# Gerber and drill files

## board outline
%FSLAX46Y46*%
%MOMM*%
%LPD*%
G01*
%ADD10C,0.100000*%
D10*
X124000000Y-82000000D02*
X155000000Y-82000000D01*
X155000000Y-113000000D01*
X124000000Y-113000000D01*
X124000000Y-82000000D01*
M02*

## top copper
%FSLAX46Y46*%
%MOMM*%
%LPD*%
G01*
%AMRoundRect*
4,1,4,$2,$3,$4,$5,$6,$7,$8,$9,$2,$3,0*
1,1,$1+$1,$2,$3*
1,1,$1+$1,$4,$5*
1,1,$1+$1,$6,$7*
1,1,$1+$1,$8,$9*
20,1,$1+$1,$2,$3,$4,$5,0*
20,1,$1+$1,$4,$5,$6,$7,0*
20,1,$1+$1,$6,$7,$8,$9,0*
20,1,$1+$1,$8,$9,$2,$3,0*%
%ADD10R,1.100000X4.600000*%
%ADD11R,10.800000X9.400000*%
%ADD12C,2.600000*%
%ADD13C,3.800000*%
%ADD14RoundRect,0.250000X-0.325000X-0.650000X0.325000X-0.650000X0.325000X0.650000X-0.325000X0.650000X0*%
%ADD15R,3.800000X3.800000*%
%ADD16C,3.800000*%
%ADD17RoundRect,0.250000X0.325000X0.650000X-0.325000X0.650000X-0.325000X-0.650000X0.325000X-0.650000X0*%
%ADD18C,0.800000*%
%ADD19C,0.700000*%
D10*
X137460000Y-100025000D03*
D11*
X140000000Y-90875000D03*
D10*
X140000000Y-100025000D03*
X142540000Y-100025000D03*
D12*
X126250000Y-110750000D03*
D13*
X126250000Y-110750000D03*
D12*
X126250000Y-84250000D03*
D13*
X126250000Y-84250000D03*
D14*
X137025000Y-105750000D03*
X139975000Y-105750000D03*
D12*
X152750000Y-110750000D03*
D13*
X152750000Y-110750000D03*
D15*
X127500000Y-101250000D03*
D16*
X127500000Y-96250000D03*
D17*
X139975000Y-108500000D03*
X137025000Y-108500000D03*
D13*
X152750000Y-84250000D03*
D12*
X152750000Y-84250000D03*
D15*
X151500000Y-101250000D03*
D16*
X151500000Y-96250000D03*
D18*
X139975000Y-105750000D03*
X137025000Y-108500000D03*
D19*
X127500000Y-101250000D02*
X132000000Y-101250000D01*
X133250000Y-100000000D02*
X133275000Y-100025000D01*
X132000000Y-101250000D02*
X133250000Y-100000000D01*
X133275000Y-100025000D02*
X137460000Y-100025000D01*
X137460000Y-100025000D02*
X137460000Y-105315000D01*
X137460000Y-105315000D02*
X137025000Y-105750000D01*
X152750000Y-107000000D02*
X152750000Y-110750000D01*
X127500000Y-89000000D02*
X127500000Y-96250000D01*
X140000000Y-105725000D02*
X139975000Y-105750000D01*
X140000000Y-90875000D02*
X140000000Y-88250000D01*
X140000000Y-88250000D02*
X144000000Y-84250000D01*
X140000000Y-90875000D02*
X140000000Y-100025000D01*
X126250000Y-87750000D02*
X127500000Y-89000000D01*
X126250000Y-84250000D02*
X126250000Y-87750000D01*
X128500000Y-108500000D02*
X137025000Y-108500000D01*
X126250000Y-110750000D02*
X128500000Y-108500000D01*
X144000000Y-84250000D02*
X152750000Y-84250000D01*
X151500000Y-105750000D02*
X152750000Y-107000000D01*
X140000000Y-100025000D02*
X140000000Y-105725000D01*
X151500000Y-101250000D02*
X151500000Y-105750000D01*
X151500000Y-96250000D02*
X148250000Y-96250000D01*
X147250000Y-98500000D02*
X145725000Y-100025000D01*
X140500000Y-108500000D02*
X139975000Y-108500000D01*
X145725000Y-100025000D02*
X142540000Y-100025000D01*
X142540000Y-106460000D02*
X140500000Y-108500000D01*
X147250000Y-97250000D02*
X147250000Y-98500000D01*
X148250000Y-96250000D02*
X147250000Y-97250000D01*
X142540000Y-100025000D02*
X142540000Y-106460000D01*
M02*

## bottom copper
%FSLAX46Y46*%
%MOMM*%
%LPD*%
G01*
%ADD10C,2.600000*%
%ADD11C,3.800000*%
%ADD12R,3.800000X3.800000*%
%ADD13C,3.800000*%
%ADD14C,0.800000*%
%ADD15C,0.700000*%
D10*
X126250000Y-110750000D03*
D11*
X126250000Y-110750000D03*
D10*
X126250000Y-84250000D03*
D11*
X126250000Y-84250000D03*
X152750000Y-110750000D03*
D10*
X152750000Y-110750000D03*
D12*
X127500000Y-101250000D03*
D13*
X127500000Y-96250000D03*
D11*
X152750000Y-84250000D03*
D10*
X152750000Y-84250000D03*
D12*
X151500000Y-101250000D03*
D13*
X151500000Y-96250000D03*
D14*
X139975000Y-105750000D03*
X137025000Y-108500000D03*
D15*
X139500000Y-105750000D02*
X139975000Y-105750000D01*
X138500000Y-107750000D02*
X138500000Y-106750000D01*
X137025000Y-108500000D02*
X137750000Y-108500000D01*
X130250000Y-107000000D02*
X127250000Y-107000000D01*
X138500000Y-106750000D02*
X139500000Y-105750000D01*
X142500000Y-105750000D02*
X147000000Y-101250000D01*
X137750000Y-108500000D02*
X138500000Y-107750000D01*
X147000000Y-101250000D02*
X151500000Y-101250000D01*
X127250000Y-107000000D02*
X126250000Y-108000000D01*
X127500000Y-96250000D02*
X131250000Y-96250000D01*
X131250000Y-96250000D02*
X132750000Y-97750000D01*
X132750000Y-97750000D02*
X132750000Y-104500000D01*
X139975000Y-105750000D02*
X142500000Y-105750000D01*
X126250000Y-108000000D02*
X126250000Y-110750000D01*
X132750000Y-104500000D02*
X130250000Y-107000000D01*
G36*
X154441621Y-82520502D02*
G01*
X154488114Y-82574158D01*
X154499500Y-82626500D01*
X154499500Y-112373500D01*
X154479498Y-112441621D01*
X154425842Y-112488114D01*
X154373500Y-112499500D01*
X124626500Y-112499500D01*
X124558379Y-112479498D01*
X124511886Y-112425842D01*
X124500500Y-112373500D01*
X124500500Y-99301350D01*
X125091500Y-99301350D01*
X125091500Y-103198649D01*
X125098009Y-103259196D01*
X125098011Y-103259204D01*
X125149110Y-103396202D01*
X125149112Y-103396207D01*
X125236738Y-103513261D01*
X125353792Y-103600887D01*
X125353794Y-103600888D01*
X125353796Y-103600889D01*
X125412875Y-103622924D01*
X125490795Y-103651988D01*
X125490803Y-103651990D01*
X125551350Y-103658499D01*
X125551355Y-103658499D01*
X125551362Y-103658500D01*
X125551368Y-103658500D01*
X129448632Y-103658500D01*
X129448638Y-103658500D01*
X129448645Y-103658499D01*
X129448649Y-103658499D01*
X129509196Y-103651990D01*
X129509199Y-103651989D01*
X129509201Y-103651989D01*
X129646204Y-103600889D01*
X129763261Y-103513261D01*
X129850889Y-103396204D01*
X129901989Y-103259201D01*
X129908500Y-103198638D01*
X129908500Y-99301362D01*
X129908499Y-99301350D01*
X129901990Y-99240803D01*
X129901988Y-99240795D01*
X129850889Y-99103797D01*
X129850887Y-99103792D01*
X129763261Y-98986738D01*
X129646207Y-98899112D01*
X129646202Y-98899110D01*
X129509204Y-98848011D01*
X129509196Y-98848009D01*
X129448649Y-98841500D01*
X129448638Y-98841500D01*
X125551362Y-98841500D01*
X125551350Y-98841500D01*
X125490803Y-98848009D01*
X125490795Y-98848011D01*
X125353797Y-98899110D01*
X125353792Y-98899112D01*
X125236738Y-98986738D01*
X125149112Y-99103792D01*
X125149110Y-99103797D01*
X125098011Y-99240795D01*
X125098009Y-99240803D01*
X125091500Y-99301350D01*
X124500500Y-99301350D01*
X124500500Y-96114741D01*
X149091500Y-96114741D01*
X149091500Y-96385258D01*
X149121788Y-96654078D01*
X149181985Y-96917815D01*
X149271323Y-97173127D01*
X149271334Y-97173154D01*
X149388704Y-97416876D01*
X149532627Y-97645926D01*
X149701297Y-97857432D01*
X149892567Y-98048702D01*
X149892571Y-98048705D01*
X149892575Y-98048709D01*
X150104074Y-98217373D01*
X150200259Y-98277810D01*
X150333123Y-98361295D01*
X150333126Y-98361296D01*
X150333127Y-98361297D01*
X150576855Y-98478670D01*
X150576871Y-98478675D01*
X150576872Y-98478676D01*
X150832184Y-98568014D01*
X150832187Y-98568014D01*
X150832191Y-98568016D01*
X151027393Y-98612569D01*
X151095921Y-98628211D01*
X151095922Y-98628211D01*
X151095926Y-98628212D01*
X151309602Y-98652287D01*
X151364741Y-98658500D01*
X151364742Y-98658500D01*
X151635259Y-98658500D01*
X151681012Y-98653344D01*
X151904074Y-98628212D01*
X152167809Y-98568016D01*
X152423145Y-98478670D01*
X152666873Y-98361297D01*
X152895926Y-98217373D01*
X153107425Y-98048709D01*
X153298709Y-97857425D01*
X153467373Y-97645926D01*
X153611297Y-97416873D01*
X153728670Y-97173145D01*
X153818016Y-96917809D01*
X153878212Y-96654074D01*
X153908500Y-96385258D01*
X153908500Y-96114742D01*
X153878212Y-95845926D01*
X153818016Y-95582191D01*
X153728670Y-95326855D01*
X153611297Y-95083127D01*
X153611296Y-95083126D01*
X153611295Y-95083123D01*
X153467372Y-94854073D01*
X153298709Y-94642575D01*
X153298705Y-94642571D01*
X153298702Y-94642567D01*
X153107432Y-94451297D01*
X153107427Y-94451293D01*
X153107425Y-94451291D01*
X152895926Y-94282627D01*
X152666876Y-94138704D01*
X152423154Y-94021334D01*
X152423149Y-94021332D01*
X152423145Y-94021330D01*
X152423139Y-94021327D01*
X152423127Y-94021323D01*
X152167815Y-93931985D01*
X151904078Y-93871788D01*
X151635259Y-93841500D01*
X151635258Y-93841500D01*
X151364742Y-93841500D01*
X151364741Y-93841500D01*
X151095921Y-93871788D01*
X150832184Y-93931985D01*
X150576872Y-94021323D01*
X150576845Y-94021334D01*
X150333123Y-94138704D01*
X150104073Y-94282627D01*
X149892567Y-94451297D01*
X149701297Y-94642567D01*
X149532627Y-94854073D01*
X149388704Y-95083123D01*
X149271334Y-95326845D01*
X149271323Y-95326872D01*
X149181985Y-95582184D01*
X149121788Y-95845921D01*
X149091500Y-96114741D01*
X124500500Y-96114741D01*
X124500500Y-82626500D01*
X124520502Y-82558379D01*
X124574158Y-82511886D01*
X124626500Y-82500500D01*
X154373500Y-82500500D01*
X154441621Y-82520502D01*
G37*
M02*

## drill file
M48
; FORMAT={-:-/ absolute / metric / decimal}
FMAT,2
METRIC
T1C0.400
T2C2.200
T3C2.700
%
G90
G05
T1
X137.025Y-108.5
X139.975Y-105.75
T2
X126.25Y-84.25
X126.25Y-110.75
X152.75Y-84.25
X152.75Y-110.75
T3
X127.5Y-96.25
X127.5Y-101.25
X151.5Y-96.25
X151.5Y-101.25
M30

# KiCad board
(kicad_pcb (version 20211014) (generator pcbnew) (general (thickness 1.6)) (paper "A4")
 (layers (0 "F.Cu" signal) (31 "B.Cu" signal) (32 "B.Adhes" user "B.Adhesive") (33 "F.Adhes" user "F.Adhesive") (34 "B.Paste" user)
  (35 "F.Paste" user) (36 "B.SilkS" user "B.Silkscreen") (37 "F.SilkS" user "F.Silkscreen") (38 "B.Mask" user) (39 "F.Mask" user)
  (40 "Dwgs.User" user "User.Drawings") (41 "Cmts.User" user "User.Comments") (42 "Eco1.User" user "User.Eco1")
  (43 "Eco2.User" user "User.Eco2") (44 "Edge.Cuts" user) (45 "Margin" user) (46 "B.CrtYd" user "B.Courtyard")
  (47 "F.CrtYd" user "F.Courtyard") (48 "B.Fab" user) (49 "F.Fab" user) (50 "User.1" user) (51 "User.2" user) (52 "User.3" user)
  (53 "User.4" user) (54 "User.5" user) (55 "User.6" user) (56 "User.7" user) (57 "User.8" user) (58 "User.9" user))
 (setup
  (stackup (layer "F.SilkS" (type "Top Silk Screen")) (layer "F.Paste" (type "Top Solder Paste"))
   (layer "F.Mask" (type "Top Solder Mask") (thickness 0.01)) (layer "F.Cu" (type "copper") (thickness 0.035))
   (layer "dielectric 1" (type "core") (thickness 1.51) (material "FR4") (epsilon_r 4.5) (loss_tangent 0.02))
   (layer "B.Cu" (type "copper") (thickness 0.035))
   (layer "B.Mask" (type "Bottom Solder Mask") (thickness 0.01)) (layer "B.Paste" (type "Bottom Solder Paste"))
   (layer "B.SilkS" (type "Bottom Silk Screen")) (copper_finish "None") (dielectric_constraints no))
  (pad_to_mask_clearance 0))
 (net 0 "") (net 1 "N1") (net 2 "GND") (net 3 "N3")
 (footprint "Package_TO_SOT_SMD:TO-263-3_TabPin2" (layer "F.Cu") (at 140 94.25 90)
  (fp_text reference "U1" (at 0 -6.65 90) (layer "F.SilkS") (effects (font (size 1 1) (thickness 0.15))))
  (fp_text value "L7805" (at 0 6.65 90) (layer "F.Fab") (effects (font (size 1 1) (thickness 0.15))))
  (pad "" smd rect (at 5.8 2.775 90) (size 4.55 5.25) (layers "F.Paste"))
  (pad "" smd rect (at 0.95 2.775 90) (size 4.55 5.25) (layers "F.Paste"))
  (pad "" smd rect (at 0.95 -2.775 90) (size 4.55 5.25) (layers "F.Paste"))
  (pad "" smd rect (at 5.8 -2.775 90) (size 4.55 5.25) (layers "F.Paste"))
  (pad "1" smd rect (at -5.775 -2.54 90) (size 4.6 1.1) (layers "F.Cu" "F.Paste" "F.Mask") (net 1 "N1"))
  (pad "2" smd rect (at 3.375 0 90) (size 9.4 10.8) (layers "F.Cu" "F.Mask") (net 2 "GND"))
  (pad "2" smd rect (at -5.775 0 90) (size 4.6 1.1) (layers "F.Cu" "F.Paste" "F.Mask") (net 2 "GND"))
  (pad "3" smd rect (at -5.775 2.54 90) (size 4.6 1.1) (layers "F.Cu" "F.Paste" "F.Mask") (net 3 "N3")))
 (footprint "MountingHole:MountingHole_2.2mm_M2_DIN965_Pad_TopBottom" (layer "F.Cu") (at 126.25 110.75)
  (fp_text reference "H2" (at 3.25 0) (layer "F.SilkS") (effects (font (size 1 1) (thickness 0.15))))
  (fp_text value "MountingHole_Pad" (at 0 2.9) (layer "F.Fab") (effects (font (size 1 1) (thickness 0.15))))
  (pad "1" thru_hole circle (at 0 0) (size 2.6 2.6) (drill 2.2) (layers *.Cu *.Mask) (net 2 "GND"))
  (pad "1" connect circle (at 0 0) (size 3.8 3.8) (layers "F.Cu" "F.Mask") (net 2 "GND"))
  (pad "1" connect circle (at 0 0) (size 3.8 3.8) (layers "B.Cu" "B.Mask") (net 2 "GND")))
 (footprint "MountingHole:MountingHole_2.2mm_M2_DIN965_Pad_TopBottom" (layer "F.Cu") (at 126.25 84.25)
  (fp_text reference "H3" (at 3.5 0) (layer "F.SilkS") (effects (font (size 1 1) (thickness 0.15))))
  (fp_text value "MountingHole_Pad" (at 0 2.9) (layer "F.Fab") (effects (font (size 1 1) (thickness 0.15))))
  (pad "1" thru_hole circle (at 0 0) (size 2.6 2.6) (drill 2.2) (layers *.Cu *.Mask) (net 2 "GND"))
  (pad "1" connect circle (at 0 0) (size 3.8 3.8) (layers "F.Cu" "F.Mask") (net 2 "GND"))
  (pad "1" connect circle (at 0 0) (size 3.8 3.8) (layers "B.Cu" "B.Mask") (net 2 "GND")))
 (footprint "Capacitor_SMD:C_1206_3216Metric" (layer "F.Cu") (at 138.5 105.75)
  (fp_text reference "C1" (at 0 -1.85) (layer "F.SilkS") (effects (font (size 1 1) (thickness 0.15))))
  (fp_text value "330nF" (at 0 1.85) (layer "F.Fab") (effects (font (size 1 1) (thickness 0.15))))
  (pad "1" smd roundrect (at -1.475 0) (size 1.15 1.8) (layers "F.Cu" "F.Paste" "F.Mask") (roundrect_rratio 0.217391) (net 1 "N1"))
  (pad "2" smd roundrect (at 1.475 0) (size 1.15 1.8) (layers "F.Cu" "F.Paste" "F.Mask") (roundrect_rratio 0.217391) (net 2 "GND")))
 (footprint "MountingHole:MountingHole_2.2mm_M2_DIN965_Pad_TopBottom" (layer "F.Cu") (at 152.75 110.75)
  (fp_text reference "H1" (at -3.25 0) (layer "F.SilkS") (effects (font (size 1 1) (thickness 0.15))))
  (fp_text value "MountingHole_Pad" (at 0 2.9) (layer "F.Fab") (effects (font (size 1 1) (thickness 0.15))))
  (pad "1" connect circle (at 0 0) (size 3.8 3.8) (layers "B.Cu" "B.Mask") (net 2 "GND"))
  (pad "1" thru_hole circle (at 0 0) (size 2.6 2.6) (drill 2.2) (layers *.Cu *.Mask) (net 2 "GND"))
  (pad "1" connect circle (at 0 0) (size 3.8 3.8) (layers "F.Cu" "F.Mask") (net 2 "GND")))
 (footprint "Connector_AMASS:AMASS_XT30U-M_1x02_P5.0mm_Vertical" (layer "F.Cu") (at 127.5 101.25 90)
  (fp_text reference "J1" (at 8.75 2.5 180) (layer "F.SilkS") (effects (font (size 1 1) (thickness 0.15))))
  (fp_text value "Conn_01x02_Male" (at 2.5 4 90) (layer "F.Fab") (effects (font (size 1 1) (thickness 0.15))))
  (pad "1" thru_hole rect (at 0 0 90) (size 3.8 3.8) (drill 2.7) (layers *.Cu *.Mask) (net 1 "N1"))
  (pad "2" thru_hole circle (at 5 0 90) (size 3.8 3.8) (drill 2.7) (layers *.Cu *.Mask) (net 2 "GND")))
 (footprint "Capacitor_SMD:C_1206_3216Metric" (layer "F.Cu") (at 138.5 108.5 180)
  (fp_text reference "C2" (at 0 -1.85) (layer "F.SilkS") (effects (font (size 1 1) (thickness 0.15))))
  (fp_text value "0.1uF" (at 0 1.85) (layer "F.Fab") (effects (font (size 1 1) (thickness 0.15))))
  (pad "1" smd roundrect (at -1.475 0 180) (size 1.15 1.8) (layers "F.Cu" "F.Paste" "F.Mask") (roundrect_rratio 0.217391) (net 3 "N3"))
  (pad "2" smd roundrect (at 1.475 0 180) (size 1.15 1.8) (layers "F.Cu" "F.Paste" "F.Mask") (roundrect_rratio 0.217391) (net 2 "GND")))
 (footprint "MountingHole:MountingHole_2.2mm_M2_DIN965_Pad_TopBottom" (layer "F.Cu") (at 152.75 84.25)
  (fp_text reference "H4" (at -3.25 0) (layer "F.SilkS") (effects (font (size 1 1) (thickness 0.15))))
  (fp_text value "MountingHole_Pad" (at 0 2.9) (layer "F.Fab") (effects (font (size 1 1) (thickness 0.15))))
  (pad "1" connect circle (at 0 0) (size 3.8 3.8) (layers "B.Cu" "B.Mask") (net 2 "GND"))
  (pad "1" connect circle (at 0 0) (size 3.8 3.8) (layers "F.Cu" "F.Mask") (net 2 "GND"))
  (pad "1" thru_hole circle (at 0 0) (size 2.6 2.6) (drill 2.2) (layers *.Cu *.Mask) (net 2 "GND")))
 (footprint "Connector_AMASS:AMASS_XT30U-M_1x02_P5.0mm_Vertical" (layer "F.Cu") (at 151.5 101.25 90)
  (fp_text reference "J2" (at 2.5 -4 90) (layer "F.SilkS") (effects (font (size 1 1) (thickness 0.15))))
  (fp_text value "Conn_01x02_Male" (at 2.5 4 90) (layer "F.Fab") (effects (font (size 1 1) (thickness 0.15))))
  (pad "1" thru_hole rect (at 0 0 90) (size 3.8 3.8) (drill 2.7) (layers *.Cu *.Mask) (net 2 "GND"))
  (pad "2" thru_hole circle (at 5 0 90) (size 3.8 3.8) (drill 2.7) (layers *.Cu *.Mask) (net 3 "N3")))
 (gr_rect (start 124 82) (end 155 113) (layer "Edge.Cuts") (width 0.1) (fill none))
 (segment (start 127.5 101.25) (end 132 101.25) (width 0.7) (layer "F.Cu") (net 1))
 (segment (start 133.25 100) (end 133.275 100.025) (width 0.7) (layer "F.Cu") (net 1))
 (segment (start 132 101.25) (end 133.25 100) (width 0.7) (layer "F.Cu") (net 1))
 (segment (start 133.275 100.025) (end 137.46 100.025) (width 0.7) (layer "F.Cu") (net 1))
 (segment (start 137.46 100.025) (end 137.46 105.315) (width 0.7) (layer "F.Cu") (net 1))
 (segment (start 137.46 105.315) (end 137.025 105.75) (width 0.7) (layer "F.Cu") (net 1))
 (segment (start 152.75 107) (end 152.75 110.75) (width 0.7) (layer "F.Cu") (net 2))
 (segment (start 127.5 89) (end 127.5 96.25) (width 0.7) (layer "F.Cu") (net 2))
 (segment (start 140 105.725) (end 139.975 105.75) (width 0.7) (layer "F.Cu") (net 2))
 (segment (start 140 90.875) (end 140 88.25) (width 0.7) (layer "F.Cu") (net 2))
 (segment (start 140 88.25) (end 144 84.25) (width 0.7) (layer "F.Cu") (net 2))
 (segment (start 140 90.875) (end 140 100.025) (width 0.7) (layer "F.Cu") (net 2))
 (segment (start 126.25 87.75) (end 127.5 89) (width 0.7) (layer "F.Cu") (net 2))
 (segment (start 126.25 84.25) (end 126.25 87.75) (width 0.7) (layer "F.Cu") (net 2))
 (segment (start 128.5 108.5) (end 137.025 108.5) (width 0.7) (layer "F.Cu") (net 2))
 (segment (start 126.25 110.75) (end 128.5 108.5) (width 0.7) (layer "F.Cu") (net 2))
 (segment (start 144 84.25) (end 152.75 84.25) (width 0.7) (layer "F.Cu") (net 2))
 (segment (start 151.5 105.75) (end 152.75 107) (width 0.7) (layer "F.Cu") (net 2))
 (segment (start 140 100.025) (end 140 105.725) (width 0.7) (layer "F.Cu") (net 2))
 (segment (start 151.5 101.25) (end 151.5 105.75) (width 0.7) (layer "F.Cu") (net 2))
 (via (at 139.975 105.75) (size 0.8) (drill 0.4) (layers "F.Cu" "B.Cu") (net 2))
 (via (at 137.025 108.5) (size 0.8) (drill 0.4) (layers "F.Cu" "B.Cu") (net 2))
 (segment (start 139.5 105.75) (end 139.975 105.75) (width 0.7) (layer "B.Cu") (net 2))
 (segment (start 138.5 107.75) (end 138.5 106.75) (width 0.7) (layer "B.Cu") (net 2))
 (segment (start 137.025 108.5) (end 137.75 108.5) (width 0.7) (layer "B.Cu") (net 2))
 (segment (start 130.25 107) (end 127.25 107) (width 0.7) (layer "B.Cu") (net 2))
 (segment (start 138.5 106.75) (end 139.5 105.75) (width 0.7) (layer "B.Cu") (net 2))
 (segment (start 142.5 105.75) (end 147 101.25) (width 0.7) (layer "B.Cu") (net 2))
 (segment (start 137.75 108.5) (end 138.5 107.75) (width 0.7) (layer "B.Cu") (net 2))
 (segment (start 147 101.25) (end 151.5 101.25) (width 0.7) (layer "B.Cu") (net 2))
 (segment (start 127.25 107) (end 126.25 108) (width 0.7) (layer "B.Cu") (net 2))
 (segment (start 127.5 96.25) (end 131.25 96.25) (width 0.7) (layer "B.Cu") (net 2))
 (segment (start 131.25 96.25) (end 132.75 97.75) (width 0.7) (layer "B.Cu") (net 2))
 (segment (start 132.75 97.75) (end 132.75 104.5) (width 0.7) (layer "B.Cu") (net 2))
 (segment (start 139.975 105.75) (end 142.5 105.75) (width 0.7) (layer "B.Cu") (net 2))
 (segment (start 126.25 108) (end 126.25 110.75) (width 0.7) (layer "B.Cu") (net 2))
 (segment (start 132.75 104.5) (end 130.25 107) (width 0.7) (layer "B.Cu") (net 2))
 (segment (start 151.5 96.25) (end 148.25 96.25) (width 0.7) (layer "F.Cu") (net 3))
 (segment (start 147.25 98.5) (end 145.725 100.025) (width 0.7) (layer "F.Cu") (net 3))
 (segment (start 140.5 108.5) (end 139.975 108.5) (width 0.7) (layer "F.Cu") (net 3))
 (segment (start 145.725 100.025) (end 142.54 100.025) (width 0.7) (layer "F.Cu") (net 3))
 (segment (start 142.54 106.46) (end 140.5 108.5) (width 0.7) (layer "F.Cu") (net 3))
 (segment (start 147.25 97.25) (end 147.25 98.5) (width 0.7) (layer "F.Cu") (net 3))
 (segment (start 148.25 96.25) (end 147.25 97.25) (width 0.7) (layer "F.Cu") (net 3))
 (segment (start 142.54 100.025) (end 142.54 106.46) (width 0.7) (layer "F.Cu") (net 3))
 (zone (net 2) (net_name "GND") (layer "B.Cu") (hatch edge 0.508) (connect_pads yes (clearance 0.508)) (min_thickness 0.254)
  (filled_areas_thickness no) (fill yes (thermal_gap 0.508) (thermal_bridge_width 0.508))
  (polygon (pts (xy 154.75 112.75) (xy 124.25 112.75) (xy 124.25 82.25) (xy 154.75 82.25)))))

